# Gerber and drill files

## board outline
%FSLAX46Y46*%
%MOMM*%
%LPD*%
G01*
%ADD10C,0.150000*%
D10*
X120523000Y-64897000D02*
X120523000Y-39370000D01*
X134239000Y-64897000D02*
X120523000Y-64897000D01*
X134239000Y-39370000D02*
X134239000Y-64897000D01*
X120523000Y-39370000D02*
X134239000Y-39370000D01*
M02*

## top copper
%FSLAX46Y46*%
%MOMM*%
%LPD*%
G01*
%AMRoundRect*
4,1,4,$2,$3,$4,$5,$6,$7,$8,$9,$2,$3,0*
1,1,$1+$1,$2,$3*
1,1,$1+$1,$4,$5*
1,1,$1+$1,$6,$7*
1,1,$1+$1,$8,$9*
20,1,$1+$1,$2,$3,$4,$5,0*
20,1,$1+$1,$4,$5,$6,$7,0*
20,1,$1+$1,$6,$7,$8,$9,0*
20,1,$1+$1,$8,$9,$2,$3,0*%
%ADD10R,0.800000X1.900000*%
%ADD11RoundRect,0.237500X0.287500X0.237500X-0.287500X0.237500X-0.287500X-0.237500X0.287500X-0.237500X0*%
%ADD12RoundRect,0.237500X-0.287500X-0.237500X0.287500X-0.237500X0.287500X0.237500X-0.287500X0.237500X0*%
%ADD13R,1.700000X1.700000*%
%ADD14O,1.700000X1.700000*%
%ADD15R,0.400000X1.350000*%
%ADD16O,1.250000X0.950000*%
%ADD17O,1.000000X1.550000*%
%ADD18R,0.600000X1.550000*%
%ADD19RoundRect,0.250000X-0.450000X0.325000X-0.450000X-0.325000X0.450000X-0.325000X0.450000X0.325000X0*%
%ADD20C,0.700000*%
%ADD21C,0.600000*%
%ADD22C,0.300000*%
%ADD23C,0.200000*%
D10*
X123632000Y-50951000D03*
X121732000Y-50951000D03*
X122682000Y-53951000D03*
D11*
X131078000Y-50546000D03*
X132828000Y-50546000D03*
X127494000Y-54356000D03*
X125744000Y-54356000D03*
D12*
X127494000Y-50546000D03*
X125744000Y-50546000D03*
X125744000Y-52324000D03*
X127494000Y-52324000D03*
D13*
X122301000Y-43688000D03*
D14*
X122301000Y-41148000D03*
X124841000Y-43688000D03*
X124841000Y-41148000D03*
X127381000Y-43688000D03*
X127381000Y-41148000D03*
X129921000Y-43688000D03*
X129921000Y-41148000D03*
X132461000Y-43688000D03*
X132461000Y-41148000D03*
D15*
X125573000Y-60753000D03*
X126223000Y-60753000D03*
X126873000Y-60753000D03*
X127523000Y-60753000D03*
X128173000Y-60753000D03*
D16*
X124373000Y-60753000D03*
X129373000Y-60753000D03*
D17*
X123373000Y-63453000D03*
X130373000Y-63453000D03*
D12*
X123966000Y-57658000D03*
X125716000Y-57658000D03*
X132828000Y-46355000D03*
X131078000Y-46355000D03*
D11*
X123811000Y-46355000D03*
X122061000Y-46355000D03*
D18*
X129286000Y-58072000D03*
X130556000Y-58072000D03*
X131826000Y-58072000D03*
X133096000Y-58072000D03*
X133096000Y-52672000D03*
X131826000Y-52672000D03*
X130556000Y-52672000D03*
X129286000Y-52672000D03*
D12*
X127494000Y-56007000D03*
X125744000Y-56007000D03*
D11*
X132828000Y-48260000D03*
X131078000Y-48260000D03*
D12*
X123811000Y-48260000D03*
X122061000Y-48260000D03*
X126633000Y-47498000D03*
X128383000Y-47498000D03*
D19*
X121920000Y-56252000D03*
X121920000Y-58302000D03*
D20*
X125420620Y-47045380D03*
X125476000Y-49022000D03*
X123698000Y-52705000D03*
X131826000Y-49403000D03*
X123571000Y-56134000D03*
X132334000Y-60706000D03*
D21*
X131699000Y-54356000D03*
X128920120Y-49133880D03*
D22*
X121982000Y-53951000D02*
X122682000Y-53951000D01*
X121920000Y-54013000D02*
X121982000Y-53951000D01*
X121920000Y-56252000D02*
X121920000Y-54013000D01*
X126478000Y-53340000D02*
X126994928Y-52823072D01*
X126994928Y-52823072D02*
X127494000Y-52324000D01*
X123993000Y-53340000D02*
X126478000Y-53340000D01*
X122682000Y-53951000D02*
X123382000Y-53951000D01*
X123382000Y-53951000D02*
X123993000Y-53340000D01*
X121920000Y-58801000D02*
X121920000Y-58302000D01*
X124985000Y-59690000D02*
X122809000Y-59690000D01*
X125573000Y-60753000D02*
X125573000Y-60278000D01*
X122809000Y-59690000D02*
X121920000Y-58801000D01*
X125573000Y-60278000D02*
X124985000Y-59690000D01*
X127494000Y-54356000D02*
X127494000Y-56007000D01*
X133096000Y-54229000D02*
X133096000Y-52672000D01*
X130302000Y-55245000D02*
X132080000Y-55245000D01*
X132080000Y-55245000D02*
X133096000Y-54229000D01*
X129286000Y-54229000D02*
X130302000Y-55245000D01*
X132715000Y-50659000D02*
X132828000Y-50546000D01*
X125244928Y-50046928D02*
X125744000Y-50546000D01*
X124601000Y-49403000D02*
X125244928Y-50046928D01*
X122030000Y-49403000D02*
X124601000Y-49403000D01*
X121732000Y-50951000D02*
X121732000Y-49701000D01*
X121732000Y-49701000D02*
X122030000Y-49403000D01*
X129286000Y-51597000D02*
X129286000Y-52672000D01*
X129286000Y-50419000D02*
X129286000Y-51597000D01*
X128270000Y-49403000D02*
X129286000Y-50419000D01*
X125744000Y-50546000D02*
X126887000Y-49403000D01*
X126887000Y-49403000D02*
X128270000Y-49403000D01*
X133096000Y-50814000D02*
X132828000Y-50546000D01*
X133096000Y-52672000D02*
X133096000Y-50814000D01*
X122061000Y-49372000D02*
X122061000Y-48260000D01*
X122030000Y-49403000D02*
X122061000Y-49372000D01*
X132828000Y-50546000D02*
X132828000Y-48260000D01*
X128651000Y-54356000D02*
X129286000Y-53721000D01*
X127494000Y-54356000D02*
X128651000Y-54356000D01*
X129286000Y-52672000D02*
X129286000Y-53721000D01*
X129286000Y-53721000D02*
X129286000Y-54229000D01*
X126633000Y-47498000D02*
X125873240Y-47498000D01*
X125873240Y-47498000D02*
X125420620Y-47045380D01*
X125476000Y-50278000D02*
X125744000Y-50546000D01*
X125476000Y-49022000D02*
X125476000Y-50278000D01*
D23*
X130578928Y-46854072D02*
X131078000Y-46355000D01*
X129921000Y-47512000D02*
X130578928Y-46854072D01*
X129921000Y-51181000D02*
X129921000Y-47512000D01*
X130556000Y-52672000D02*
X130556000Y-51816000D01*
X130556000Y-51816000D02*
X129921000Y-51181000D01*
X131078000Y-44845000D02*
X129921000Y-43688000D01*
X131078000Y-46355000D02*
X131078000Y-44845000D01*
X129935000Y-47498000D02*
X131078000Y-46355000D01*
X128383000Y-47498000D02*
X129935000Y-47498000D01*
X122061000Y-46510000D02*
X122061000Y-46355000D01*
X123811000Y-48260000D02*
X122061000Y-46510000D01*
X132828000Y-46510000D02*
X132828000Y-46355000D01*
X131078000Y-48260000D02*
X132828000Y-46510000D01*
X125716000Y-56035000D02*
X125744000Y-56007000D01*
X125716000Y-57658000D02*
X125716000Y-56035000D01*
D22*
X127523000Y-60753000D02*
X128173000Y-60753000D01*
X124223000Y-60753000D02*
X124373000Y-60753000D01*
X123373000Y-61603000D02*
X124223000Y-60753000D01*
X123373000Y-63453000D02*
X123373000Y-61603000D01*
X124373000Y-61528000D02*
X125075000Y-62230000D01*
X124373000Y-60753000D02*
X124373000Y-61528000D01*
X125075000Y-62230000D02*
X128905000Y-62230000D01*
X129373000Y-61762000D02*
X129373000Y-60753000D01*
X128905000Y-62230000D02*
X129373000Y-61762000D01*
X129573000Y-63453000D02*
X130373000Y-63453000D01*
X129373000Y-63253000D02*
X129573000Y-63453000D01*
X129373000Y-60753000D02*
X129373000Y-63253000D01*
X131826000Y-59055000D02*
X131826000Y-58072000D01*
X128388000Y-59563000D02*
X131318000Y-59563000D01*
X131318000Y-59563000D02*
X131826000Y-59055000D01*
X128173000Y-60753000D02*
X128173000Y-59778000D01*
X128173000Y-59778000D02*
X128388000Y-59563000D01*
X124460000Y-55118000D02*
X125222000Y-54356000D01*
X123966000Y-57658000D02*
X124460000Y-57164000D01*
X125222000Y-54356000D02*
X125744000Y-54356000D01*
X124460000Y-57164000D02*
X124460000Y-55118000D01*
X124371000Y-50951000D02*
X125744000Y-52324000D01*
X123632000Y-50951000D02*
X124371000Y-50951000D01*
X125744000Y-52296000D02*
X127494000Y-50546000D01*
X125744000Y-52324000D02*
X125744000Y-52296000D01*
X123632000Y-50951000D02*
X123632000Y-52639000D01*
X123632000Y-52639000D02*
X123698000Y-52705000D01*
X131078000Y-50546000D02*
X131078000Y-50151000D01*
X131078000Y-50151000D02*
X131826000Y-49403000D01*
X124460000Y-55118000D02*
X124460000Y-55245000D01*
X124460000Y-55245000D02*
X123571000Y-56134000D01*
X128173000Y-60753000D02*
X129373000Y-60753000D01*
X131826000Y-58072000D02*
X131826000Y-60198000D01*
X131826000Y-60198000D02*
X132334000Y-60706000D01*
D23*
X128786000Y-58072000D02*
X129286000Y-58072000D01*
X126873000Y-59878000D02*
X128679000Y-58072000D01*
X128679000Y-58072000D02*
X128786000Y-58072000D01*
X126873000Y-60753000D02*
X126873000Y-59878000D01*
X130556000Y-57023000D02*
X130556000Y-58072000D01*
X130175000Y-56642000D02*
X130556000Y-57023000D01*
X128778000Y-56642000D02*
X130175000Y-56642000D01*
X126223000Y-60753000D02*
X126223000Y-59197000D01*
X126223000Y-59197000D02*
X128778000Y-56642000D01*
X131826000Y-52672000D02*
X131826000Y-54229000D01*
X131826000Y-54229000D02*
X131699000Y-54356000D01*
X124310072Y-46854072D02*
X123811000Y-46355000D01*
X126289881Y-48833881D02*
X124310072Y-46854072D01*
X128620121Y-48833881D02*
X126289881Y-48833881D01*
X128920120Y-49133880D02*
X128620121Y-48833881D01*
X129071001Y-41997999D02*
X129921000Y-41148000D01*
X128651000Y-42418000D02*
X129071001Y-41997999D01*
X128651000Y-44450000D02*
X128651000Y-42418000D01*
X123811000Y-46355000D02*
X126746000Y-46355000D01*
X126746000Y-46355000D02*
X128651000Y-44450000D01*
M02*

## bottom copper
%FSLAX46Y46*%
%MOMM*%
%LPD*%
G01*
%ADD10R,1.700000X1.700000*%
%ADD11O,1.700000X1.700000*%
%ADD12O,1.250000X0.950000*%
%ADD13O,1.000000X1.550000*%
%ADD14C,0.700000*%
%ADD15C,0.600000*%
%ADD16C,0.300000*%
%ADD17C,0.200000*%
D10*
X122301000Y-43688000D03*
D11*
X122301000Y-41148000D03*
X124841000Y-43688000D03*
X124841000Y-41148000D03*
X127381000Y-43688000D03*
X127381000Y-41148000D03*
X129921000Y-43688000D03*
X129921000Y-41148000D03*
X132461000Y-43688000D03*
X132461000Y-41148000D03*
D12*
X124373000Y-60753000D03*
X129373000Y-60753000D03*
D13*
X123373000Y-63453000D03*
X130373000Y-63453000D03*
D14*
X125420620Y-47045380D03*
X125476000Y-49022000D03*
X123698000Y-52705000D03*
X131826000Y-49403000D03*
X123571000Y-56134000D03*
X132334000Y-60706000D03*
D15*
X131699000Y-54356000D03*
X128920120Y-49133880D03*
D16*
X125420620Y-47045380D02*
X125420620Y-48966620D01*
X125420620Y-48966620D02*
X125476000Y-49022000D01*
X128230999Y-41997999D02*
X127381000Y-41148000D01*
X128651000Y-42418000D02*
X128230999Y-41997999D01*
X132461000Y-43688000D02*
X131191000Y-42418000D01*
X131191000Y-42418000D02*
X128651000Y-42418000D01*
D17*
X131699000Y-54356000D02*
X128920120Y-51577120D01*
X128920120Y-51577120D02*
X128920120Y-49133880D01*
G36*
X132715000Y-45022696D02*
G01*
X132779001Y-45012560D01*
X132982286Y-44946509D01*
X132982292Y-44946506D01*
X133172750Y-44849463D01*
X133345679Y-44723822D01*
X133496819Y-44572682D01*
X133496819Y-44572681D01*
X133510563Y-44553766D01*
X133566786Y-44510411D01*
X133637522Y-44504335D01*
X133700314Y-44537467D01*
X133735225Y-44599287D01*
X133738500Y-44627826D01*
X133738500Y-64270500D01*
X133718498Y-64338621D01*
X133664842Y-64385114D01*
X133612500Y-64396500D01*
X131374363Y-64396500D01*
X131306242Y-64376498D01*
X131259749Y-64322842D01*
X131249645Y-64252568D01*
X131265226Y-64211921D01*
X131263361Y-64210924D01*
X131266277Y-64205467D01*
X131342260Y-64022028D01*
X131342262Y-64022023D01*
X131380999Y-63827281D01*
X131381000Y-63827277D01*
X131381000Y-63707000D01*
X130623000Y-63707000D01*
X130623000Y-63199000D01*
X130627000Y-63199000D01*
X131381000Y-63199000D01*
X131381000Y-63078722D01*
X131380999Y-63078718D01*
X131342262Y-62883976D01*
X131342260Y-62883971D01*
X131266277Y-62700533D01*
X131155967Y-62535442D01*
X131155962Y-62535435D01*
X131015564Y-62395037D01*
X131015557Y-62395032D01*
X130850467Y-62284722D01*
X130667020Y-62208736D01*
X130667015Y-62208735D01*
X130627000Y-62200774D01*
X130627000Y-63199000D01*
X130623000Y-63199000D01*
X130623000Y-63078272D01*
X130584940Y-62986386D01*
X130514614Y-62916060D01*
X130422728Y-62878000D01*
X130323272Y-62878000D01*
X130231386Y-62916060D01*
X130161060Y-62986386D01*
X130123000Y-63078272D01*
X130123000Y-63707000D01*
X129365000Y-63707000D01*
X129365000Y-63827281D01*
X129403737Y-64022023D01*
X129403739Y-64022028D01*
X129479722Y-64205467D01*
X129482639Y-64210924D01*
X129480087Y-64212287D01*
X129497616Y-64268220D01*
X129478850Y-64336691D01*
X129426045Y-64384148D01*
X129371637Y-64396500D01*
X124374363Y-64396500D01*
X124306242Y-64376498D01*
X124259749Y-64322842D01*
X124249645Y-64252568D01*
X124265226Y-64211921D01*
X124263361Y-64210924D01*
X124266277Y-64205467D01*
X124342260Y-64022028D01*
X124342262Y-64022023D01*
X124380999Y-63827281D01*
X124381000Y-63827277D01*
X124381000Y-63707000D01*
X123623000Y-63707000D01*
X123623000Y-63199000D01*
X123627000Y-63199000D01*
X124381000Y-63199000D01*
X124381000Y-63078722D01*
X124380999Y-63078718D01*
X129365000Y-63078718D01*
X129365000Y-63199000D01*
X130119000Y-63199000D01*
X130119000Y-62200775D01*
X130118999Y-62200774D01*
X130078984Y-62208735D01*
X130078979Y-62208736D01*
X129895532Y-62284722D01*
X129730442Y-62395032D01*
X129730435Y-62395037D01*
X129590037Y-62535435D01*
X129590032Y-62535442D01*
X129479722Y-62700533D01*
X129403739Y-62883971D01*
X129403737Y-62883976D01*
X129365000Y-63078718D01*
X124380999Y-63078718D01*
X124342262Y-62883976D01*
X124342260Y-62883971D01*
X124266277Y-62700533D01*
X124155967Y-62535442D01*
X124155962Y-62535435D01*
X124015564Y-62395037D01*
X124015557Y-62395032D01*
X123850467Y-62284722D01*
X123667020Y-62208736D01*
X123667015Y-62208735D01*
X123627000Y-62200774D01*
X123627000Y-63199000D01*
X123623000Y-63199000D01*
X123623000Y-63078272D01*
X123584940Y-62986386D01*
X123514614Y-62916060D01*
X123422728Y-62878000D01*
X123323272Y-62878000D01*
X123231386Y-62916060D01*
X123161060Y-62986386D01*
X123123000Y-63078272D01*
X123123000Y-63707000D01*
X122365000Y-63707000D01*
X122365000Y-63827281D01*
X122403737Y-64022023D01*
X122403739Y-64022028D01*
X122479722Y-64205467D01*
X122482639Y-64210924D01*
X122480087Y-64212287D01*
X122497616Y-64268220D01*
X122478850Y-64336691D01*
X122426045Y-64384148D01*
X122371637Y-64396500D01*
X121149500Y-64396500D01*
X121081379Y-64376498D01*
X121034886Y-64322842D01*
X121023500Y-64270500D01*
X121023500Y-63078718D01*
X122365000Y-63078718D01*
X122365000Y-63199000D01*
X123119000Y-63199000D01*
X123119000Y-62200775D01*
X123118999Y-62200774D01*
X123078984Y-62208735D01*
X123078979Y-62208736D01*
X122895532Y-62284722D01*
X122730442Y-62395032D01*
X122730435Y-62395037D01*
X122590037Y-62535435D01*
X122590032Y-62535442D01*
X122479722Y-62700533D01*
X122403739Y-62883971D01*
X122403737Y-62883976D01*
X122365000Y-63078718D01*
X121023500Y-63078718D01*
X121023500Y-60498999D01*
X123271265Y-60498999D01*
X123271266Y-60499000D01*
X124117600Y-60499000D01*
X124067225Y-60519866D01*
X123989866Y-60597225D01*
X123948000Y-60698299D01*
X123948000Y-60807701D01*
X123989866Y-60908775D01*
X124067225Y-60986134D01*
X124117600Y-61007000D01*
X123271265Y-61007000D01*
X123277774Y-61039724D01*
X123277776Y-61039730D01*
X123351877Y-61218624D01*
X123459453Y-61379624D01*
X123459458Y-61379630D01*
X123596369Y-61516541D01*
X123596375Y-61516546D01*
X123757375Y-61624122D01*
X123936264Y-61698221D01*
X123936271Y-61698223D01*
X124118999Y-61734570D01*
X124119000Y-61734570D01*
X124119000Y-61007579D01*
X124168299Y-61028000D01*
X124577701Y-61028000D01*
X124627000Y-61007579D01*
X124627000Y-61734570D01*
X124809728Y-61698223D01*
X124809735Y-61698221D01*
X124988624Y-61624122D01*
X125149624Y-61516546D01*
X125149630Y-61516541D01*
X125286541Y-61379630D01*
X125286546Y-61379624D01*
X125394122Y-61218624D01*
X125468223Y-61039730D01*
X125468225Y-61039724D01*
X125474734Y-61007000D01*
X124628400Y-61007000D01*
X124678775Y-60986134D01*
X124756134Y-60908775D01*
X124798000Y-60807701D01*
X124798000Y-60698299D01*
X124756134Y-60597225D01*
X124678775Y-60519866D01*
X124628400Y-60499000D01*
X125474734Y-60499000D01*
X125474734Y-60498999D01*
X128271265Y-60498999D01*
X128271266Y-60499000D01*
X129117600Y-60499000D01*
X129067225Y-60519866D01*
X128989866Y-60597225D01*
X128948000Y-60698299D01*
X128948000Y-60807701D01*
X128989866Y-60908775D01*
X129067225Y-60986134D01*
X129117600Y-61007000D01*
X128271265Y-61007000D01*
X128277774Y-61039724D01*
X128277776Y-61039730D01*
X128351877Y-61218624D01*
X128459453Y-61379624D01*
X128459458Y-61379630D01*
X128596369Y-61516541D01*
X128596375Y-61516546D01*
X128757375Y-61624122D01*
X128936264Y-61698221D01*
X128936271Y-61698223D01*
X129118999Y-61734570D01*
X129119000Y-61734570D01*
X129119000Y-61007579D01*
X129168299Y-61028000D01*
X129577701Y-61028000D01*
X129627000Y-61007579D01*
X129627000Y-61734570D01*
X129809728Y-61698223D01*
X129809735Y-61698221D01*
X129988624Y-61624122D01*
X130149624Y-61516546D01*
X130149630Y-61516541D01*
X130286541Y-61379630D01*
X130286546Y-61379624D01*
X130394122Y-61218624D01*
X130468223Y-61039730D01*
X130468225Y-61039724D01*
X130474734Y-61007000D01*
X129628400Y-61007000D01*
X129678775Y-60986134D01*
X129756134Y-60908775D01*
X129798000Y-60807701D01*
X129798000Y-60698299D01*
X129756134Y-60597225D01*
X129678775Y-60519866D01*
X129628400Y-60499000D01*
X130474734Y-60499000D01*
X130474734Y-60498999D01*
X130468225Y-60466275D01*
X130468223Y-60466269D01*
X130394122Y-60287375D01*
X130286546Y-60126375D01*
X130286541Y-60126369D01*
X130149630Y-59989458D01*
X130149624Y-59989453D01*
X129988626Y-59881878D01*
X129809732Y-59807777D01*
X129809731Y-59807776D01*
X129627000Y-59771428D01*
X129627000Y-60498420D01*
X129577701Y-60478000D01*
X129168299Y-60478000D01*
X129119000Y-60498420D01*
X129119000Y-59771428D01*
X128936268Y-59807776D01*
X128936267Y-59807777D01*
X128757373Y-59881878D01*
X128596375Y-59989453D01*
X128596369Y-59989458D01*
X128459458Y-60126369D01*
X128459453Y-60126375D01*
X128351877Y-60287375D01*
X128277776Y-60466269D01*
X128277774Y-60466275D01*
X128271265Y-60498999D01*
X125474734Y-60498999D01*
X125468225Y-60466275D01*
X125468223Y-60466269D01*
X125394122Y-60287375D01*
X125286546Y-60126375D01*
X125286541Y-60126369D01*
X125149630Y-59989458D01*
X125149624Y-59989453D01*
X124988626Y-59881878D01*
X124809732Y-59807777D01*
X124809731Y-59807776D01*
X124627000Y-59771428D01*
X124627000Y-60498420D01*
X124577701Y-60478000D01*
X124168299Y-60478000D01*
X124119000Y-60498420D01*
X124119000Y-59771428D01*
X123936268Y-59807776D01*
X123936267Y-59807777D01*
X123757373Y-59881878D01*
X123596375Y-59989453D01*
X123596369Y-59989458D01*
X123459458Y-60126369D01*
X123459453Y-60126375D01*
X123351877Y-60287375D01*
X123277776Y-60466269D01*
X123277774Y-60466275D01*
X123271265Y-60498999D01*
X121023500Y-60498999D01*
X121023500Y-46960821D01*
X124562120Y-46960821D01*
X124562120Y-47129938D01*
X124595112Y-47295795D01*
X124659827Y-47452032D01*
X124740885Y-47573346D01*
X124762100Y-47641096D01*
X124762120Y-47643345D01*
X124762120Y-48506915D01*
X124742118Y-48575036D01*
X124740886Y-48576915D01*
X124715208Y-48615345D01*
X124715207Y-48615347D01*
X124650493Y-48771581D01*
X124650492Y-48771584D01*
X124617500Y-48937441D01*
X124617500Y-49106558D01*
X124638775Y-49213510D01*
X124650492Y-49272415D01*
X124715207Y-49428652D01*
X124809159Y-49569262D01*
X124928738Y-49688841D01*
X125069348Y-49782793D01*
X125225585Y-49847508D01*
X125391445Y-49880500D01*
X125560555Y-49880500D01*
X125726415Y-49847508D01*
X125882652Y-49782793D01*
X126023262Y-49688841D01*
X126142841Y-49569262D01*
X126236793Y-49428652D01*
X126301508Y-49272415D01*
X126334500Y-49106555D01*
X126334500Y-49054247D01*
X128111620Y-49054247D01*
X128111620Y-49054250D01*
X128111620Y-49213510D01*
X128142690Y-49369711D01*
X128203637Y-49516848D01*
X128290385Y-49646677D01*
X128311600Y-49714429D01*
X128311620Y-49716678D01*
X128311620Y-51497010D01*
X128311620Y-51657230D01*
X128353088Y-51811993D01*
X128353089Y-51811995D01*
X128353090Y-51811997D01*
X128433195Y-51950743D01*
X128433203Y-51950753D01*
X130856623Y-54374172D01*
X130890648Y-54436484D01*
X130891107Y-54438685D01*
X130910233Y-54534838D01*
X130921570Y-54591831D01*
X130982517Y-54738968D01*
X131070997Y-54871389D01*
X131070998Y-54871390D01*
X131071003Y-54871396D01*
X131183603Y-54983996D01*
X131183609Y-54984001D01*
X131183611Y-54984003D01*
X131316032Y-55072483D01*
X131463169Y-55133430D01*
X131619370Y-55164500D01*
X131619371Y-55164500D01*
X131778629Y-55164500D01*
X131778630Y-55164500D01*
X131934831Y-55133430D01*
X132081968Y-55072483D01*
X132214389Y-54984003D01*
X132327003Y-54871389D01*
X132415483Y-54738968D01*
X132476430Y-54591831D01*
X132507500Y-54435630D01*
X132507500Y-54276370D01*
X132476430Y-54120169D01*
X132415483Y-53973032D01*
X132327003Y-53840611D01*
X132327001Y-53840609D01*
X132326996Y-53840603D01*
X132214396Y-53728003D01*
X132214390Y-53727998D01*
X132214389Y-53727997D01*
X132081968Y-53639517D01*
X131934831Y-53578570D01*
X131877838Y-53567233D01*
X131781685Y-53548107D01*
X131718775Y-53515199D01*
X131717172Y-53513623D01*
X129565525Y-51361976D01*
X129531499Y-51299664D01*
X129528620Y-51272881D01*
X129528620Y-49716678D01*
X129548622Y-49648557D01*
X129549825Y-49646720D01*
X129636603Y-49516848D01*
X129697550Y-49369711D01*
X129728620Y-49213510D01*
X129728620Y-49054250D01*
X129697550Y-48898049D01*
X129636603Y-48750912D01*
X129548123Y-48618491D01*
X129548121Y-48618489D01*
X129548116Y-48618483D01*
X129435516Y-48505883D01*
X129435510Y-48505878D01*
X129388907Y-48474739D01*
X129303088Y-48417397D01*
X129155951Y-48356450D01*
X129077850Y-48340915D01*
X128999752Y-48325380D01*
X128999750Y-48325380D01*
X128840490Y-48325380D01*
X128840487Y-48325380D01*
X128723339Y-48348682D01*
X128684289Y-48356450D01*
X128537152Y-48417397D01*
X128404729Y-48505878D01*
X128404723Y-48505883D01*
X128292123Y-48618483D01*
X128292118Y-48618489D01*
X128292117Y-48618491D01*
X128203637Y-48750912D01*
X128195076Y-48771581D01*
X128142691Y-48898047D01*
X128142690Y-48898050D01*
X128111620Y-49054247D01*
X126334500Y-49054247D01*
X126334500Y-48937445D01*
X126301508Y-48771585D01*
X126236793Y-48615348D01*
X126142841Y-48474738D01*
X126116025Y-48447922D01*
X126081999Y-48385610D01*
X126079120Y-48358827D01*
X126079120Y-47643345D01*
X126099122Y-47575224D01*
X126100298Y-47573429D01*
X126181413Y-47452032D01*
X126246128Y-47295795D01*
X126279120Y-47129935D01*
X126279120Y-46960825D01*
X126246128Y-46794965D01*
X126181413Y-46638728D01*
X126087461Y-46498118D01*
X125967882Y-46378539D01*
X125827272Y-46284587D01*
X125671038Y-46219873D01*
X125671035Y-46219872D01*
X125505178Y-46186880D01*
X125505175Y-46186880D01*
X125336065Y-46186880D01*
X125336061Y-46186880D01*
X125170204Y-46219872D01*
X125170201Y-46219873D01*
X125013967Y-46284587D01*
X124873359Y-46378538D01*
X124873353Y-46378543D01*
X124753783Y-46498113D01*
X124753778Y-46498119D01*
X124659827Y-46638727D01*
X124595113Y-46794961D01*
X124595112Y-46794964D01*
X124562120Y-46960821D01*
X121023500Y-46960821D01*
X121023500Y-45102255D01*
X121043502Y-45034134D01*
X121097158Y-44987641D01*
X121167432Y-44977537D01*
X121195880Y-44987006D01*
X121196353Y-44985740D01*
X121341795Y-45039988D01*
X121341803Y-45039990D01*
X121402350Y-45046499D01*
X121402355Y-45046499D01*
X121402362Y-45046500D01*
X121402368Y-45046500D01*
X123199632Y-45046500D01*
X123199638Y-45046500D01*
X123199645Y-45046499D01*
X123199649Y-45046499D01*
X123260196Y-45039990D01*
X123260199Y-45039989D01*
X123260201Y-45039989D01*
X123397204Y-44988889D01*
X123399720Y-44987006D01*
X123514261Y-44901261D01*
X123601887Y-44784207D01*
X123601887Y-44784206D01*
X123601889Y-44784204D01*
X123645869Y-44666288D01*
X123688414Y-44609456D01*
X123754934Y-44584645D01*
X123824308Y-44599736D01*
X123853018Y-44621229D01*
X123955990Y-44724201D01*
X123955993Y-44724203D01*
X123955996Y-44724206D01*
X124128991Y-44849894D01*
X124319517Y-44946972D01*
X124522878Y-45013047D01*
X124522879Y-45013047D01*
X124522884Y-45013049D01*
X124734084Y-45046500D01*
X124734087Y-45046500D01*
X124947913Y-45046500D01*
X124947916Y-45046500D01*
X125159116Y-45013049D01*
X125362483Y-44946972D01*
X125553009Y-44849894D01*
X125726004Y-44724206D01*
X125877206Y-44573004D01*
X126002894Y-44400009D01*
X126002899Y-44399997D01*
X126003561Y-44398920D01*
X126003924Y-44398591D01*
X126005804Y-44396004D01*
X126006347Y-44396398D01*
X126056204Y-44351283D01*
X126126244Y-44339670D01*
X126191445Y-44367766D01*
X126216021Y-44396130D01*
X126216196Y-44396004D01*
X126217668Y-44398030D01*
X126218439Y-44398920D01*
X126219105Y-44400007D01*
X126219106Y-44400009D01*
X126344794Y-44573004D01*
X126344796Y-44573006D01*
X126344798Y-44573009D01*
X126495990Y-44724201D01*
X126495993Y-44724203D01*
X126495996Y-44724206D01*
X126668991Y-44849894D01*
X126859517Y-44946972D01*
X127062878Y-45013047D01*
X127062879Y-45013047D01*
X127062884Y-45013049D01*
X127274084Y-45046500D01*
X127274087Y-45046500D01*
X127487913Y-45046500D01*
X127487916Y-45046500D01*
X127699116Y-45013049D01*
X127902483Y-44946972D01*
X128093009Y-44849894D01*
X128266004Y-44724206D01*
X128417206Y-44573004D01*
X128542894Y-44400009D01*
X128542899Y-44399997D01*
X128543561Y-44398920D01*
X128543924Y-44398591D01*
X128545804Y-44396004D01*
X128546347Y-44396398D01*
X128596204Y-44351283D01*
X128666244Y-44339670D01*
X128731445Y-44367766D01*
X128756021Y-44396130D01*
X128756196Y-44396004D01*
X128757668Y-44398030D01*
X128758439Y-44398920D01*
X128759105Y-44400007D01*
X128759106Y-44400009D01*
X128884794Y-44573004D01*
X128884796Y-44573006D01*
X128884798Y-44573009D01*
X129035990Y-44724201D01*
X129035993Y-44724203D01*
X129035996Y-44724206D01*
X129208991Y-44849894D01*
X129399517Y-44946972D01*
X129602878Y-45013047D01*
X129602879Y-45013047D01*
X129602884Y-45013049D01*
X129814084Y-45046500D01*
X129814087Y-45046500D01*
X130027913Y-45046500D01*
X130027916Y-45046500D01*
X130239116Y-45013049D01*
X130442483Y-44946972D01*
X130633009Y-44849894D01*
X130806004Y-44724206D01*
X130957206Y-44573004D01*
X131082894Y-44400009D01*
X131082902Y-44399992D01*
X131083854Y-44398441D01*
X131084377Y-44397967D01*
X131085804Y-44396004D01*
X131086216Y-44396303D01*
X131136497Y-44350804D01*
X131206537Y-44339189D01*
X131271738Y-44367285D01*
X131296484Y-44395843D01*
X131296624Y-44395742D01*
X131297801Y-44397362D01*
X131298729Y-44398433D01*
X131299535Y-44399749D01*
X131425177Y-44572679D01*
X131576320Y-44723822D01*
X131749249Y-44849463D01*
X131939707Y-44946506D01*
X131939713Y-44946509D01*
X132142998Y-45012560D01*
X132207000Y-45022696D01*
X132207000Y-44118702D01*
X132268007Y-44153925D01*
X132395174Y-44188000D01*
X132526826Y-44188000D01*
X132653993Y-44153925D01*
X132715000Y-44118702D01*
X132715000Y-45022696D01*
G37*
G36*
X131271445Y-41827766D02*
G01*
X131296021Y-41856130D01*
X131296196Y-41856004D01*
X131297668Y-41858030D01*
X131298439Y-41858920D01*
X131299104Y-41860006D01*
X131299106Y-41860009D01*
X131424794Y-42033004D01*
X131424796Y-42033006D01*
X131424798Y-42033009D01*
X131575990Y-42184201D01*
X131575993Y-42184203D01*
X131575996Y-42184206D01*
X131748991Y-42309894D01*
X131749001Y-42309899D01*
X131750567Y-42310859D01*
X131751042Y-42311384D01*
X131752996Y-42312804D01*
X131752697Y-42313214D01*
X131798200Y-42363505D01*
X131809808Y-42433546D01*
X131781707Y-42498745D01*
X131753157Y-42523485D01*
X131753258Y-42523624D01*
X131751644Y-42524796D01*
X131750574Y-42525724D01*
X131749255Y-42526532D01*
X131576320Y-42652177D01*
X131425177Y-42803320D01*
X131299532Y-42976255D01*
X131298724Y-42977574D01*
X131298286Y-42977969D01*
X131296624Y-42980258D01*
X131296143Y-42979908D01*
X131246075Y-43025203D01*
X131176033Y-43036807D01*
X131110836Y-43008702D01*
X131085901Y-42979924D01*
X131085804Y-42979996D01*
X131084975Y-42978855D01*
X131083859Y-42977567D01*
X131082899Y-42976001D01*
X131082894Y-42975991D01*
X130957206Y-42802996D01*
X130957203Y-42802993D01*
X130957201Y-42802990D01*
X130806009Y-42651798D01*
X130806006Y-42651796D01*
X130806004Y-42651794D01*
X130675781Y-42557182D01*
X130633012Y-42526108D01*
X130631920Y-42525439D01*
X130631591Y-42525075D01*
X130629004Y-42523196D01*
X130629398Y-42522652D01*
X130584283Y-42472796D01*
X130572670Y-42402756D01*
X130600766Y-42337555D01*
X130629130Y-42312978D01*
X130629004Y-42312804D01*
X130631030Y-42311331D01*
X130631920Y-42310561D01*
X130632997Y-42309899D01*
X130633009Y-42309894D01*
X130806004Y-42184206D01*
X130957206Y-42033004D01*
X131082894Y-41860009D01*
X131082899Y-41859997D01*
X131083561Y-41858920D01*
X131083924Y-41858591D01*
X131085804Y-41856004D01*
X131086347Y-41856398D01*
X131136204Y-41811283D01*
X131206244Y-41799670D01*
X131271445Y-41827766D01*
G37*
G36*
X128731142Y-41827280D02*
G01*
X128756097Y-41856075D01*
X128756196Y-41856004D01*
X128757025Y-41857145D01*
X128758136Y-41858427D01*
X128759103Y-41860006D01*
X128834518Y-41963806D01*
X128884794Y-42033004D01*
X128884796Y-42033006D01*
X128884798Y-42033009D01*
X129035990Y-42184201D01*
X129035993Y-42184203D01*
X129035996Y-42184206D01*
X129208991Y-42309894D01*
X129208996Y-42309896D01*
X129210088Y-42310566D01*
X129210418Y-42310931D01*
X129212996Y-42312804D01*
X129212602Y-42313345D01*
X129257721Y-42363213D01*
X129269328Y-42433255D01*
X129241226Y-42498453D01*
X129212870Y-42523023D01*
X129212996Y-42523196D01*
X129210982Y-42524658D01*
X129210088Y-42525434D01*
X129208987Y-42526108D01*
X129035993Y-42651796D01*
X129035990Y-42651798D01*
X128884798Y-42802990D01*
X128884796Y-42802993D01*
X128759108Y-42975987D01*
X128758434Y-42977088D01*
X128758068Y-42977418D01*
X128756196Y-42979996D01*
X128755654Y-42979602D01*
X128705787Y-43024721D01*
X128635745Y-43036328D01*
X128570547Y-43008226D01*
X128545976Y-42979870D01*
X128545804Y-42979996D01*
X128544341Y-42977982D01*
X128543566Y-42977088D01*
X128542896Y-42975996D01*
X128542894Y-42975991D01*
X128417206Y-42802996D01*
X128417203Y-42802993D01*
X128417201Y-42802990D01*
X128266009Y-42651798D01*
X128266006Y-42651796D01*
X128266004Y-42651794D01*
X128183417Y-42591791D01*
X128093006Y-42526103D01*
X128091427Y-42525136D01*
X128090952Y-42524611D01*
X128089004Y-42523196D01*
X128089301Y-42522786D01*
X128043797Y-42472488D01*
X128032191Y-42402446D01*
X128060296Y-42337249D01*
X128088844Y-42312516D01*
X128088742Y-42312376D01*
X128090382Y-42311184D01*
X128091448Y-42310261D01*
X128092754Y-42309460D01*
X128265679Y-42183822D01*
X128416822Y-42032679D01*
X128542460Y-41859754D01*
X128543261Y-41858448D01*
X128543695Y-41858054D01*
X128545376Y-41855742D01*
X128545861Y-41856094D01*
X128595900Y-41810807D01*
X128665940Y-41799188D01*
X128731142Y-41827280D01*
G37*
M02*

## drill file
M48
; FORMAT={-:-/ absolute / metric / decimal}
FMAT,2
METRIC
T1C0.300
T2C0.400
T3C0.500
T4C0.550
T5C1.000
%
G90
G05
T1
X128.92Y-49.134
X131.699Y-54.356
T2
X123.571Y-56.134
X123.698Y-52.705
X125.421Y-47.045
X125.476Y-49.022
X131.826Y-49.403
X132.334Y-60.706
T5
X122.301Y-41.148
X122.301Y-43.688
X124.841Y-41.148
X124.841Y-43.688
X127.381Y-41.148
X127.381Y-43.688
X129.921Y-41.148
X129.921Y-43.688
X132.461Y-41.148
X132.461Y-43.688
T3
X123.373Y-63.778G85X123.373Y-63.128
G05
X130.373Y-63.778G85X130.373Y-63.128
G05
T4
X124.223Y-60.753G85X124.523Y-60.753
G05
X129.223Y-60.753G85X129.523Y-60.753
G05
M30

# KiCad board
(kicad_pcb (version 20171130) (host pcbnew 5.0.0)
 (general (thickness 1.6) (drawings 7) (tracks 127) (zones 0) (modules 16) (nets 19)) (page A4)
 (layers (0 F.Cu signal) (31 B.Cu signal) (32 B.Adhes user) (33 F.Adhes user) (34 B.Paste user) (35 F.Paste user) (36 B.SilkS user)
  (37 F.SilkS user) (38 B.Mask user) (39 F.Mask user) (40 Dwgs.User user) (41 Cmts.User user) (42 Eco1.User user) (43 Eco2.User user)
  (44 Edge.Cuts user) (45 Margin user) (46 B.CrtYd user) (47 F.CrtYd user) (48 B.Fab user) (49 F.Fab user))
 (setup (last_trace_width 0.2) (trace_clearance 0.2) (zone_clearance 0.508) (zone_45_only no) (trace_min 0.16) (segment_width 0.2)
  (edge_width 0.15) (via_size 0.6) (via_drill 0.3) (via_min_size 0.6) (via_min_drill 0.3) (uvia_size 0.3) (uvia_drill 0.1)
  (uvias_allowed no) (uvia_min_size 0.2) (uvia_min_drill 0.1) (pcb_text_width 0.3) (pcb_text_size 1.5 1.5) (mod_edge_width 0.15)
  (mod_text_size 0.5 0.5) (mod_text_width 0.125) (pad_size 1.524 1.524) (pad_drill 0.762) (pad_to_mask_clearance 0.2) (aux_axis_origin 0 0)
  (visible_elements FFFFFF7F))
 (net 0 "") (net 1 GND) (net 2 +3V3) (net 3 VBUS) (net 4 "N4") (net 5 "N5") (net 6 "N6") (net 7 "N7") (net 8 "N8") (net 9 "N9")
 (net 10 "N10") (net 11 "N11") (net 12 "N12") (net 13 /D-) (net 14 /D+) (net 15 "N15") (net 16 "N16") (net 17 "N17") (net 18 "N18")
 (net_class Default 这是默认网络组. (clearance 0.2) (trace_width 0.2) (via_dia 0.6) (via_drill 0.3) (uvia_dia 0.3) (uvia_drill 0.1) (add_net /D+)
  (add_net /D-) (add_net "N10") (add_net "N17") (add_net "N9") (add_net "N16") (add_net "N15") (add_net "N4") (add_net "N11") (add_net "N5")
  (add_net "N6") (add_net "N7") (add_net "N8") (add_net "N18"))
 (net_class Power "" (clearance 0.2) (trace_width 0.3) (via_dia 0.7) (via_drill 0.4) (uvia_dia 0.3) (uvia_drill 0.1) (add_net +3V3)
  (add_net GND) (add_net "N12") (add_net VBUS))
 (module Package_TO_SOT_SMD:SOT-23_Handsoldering (layer F.Cu) (at 122.682 52.451 270)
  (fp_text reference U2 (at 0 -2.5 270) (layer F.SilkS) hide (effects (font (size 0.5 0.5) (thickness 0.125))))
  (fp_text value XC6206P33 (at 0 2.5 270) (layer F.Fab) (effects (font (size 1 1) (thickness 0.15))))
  (pad 1 smd rect (at -1.5 -0.95 270) (size 1.9 0.8) (layers F.Cu F.Paste F.Mask) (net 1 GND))
  (pad 2 smd rect (at -1.5 0.95 270) (size 1.9 0.8) (layers F.Cu F.Paste F.Mask) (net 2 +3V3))
  (pad 3 smd rect (at 1.5 0 270) (size 1.9 0.8) (layers F.Cu F.Paste F.Mask) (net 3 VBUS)))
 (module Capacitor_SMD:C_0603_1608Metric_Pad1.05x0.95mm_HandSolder (layer F.Cu) (at 131.953 50.546 180)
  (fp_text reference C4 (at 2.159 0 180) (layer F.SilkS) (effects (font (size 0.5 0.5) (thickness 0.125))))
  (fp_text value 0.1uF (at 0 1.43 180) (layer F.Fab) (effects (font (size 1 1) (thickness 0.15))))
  (pad 2 smd roundrect (at 0.875 0 180) (size 1.05 0.95) (layers F.Cu F.Paste F.Mask) (roundrect_rratio 0.25) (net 1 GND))
  (pad 1 smd roundrect (at -0.875 0 180) (size 1.05 0.95) (layers F.Cu F.Paste F.Mask) (roundrect_rratio 0.25) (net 2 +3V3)))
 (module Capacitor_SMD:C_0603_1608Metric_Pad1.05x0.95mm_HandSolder (layer F.Cu) (at 126.619 54.356 180)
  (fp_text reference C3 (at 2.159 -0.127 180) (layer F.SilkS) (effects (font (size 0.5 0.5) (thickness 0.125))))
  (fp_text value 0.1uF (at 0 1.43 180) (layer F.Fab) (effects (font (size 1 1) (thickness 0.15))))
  (pad 1 smd roundrect (at -0.875 0 180) (size 1.05 0.95) (layers F.Cu F.Paste F.Mask) (roundrect_rratio 0.25) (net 2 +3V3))
  (pad 2 smd roundrect (at 0.875 0 180) (size 1.05 0.95) (layers F.Cu F.Paste F.Mask) (roundrect_rratio 0.25) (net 1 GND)))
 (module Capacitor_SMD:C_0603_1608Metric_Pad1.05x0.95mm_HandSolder (layer F.Cu) (at 126.619 50.546)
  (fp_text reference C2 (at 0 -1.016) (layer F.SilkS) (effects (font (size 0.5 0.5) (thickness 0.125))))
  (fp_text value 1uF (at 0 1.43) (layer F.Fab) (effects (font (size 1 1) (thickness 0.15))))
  (pad 2 smd roundrect (at 0.875 0) (size 1.05 0.95) (layers F.Cu F.Paste F.Mask) (roundrect_rratio 0.25) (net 1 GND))
  (pad 1 smd roundrect (at -0.875 0) (size 1.05 0.95) (layers F.Cu F.Paste F.Mask) (roundrect_rratio 0.25) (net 2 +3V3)))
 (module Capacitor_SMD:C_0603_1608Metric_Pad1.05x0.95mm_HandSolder (layer F.Cu) (at 126.619 52.324)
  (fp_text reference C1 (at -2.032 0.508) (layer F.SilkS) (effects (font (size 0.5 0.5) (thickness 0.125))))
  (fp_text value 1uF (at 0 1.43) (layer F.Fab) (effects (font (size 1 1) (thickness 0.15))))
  (pad 1 smd roundrect (at -0.875 0) (size 1.05 0.95) (layers F.Cu F.Paste F.Mask) (roundrect_rratio 0.25) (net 1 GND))
  (pad 2 smd roundrect (at 0.875 0) (size 1.05 0.95) (layers F.Cu F.Paste F.Mask) (roundrect_rratio 0.25) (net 3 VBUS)))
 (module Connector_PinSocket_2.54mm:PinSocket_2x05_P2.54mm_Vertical (layer B.Cu) (at 122.301 43.688 270)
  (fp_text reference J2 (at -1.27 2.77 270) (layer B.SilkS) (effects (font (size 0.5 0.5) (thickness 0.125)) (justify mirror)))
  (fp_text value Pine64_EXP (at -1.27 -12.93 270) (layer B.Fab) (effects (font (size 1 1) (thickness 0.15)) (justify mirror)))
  (pad 1 thru_hole rect (at 0 0 270) (size 1.7 1.7) (drill 1) (layers *.Cu *.Mask) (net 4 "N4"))
  (pad 2 thru_hole oval (at -2.54 0 270) (size 1.7 1.7) (drill 1) (layers *.Cu *.Mask) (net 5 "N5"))
  (pad 3 thru_hole oval (at 0 -2.54 270) (size 1.7 1.7) (drill 1) (layers *.Cu *.Mask) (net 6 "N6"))
  (pad 4 thru_hole oval (at -2.54 -2.54 270) (size 1.7 1.7) (drill 1) (layers *.Cu *.Mask) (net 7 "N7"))
  (pad 5 thru_hole oval (at 0 -5.08 270) (size 1.7 1.7) (drill 1) (layers *.Cu *.Mask) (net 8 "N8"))
  (pad 6 thru_hole oval (at -2.54 -5.08 270) (size 1.7 1.7) (drill 1) (layers *.Cu *.Mask) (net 1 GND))
  (pad 7 thru_hole oval (at 0 -7.62 270) (size 1.7 1.7) (drill 1) (layers *.Cu *.Mask) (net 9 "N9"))
  (pad 8 thru_hole oval (at -2.54 -7.62 270) (size 1.7 1.7) (drill 1) (layers *.Cu *.Mask) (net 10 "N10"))
  (pad 9 thru_hole oval (at 0 -10.16 270) (size 1.7 1.7) (drill 1) (layers *.Cu *.Mask) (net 1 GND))
  (pad 10 thru_hole oval (at -2.54 -10.16 270) (size 1.7 1.7) (drill 1) (layers *.Cu *.Mask) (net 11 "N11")))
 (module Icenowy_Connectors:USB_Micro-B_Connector (layer F.Cu) (at 126.873 62.103)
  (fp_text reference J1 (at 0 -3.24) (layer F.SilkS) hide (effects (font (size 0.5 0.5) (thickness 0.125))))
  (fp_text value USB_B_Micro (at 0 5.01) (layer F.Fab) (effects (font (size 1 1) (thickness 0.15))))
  (pad 1 smd rect (at -1.3 -1.35 90) (size 1.35 0.4) (layers F.Cu F.Paste F.Mask) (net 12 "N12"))
  (pad 2 smd rect (at -0.65 -1.35 90) (size 1.35 0.4) (layers F.Cu F.Paste F.Mask) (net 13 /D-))
  (pad 3 smd rect (at 0 -1.35 90) (size 1.35 0.4) (layers F.Cu F.Paste F.Mask) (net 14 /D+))
  (pad 4 smd rect (at 0.65 -1.35 90) (size 1.35 0.4) (layers F.Cu F.Paste F.Mask) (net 1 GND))
  (pad 5 smd rect (at 1.3 -1.35 90) (size 1.35 0.4) (layers F.Cu F.Paste F.Mask) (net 1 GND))
  (pad 6 thru_hole oval (at -2.5 -1.35 90) (size 0.95 1.25) (drill oval 0.55 0.85) (layers *.Cu *.Mask) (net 1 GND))
  (pad 6 thru_hole oval (at 2.5 -1.35 90) (size 0.95 1.25) (drill oval 0.55 0.85) (layers *.Cu *.Mask) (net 1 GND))
  (pad 6 thru_hole oval (at -3.5 1.35 90) (size 1.55 1) (drill oval 1.15 0.5) (layers *.Cu *.Mask) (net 1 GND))
  (pad 6 thru_hole oval (at 3.5 1.35 90) (size 1.55 1) (drill oval 1.15 0.5) (layers *.Cu *.Mask) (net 1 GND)))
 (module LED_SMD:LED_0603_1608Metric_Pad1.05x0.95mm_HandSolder (layer F.Cu) (at 124.841 57.658)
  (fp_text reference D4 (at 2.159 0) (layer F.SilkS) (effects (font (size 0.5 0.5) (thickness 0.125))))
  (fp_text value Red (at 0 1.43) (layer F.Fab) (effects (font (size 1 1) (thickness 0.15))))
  (pad 1 smd roundrect (at -0.875 0) (size 1.05 0.95) (layers F.Cu F.Paste F.Mask) (roundrect_rratio 0.25) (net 1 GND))
  (pad 2 smd roundrect (at 0.875 0) (size 1.05 0.95) (layers F.Cu F.Paste F.Mask) (roundrect_rratio 0.25) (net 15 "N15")))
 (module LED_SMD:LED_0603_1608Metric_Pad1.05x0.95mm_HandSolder (layer F.Cu) (at 131.953 46.355)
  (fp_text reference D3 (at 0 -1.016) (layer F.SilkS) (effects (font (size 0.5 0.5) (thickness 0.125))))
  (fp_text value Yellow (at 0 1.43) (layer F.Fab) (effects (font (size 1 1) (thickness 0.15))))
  (pad 2 smd roundrect (at 0.875 0) (size 1.05 0.95) (layers F.Cu F.Paste F.Mask) (roundrect_rratio 0.25) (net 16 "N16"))
  (pad 1 smd roundrect (at -0.875 0) (size 1.05 0.95) (layers F.Cu F.Paste F.Mask) (roundrect_rratio 0.25) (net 9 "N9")))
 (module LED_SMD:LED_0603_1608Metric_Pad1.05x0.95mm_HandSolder (layer F.Cu) (at 122.936 46.355 180)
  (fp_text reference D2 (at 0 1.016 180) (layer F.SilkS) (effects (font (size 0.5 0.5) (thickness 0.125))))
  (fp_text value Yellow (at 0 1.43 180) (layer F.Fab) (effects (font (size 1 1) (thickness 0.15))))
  (pad 1 smd roundrect (at -0.875 0 180) (size 1.05 0.95) (layers F.Cu F.Paste F.Mask) (roundrect_rratio 0.25) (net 10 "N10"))
  (pad 2 smd roundrect (at 0.875 0 180) (size 1.05 0.95) (layers F.Cu F.Paste F.Mask) (roundrect_rratio 0.25) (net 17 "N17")))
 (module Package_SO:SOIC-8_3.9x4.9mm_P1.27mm (layer F.Cu) (at 131.191 55.372 90)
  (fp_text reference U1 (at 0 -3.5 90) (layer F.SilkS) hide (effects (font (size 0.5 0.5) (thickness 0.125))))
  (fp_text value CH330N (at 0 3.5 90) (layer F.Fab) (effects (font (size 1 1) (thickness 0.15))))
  (pad 1 smd rect (at -2.7 -1.905 90) (size 1.55 0.6) (layers F.Cu F.Paste F.Mask) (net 14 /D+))
  (pad 2 smd rect (at -2.7 -0.635 90) (size 1.55 0.6) (layers F.Cu F.Paste F.Mask) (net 13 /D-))
  (pad 3 smd rect (at -2.7 0.635 90) (size 1.55 0.6) (layers F.Cu F.Paste F.Mask) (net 1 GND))
  (pad 4 smd rect (at -2.7 1.905 90) (size 1.55 0.6) (layers F.Cu F.Paste F.Mask) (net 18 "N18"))
  (pad 5 smd rect (at 2.7 1.905 90) (size 1.55 0.6) (layers F.Cu F.Paste F.Mask) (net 2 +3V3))
  (pad 6 smd rect (at 2.7 0.635 90) (size 1.55 0.6) (layers F.Cu F.Paste F.Mask) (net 10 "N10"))
  (pad 7 smd rect (at 2.7 -0.635 90) (size 1.55 0.6) (layers F.Cu F.Paste F.Mask) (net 9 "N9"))
  (pad 8 smd rect (at 2.7 -1.905 90) (size 1.55 0.6) (layers F.Cu F.Paste F.Mask) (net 2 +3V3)))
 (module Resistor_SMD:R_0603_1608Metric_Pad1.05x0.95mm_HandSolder (layer F.Cu) (at 126.619 56.007)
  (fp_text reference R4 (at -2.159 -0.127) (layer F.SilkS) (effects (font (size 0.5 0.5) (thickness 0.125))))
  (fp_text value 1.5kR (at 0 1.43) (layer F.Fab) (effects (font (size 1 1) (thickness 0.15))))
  (pad 2 smd roundrect (at 0.875 0) (size 1.05 0.95) (layers F.Cu F.Paste F.Mask) (roundrect_rratio 0.25) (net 2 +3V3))
  (pad 1 smd roundrect (at -0.875 0) (size 1.05 0.95) (layers F.Cu F.Paste F.Mask) (roundrect_rratio 0.25) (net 15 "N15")))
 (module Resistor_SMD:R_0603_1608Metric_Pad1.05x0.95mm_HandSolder (layer F.Cu) (at 131.953 48.26 180)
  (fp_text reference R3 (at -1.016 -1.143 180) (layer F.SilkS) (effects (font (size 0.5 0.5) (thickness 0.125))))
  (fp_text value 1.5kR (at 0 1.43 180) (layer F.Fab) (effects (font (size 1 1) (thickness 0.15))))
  (pad 1 smd roundrect (at -0.875 0 180) (size 1.05 0.95) (layers F.Cu F.Paste F.Mask) (roundrect_rratio 0.25) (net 2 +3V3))
  (pad 2 smd roundrect (at 0.875 0 180) (size 1.05 0.95) (layers F.Cu F.Paste F.Mask) (roundrect_rratio 0.25) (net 16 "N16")))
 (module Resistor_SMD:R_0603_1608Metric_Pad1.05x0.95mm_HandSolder (layer F.Cu) (at 122.936 48.26)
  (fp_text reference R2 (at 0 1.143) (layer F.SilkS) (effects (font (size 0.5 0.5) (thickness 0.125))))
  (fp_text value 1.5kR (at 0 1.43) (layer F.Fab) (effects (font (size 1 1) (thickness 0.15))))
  (pad 2 smd roundrect (at 0.875 0) (size 1.05 0.95) (layers F.Cu F.Paste F.Mask) (roundrect_rratio 0.25) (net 17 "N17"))
  (pad 1 smd roundrect (at -0.875 0) (size 1.05 0.95) (layers F.Cu F.Paste F.Mask) (roundrect_rratio 0.25) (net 2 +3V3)))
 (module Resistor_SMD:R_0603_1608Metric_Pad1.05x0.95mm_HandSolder (layer F.Cu) (at 127.508 47.498)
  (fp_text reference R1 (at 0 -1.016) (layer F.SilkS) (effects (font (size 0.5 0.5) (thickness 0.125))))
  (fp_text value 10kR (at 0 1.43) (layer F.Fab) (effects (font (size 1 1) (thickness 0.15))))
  (pad 1 smd roundrect (at -0.875 0) (size 1.05 0.95) (layers F.Cu F.Paste F.Mask) (roundrect_rratio 0.25) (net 2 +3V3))
  (pad 2 smd roundrect (at 0.875 0) (size 1.05 0.95) (layers F.Cu F.Paste F.Mask) (roundrect_rratio 0.25) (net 9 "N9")))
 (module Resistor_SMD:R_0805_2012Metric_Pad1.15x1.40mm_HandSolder (layer F.Cu) (at 121.92 57.277 270)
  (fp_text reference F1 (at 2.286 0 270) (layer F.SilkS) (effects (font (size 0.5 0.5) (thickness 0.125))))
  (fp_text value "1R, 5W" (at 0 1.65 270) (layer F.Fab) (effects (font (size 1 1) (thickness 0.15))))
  (pad 1 smd roundrect (at -1.025 0 270) (size 1.15 1.4) (layers F.Cu F.Paste F.Mask) (roundrect_rratio 0.217391) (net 3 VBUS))
  (pad 2 smd roundrect (at 1.025 0 270) (size 1.15 1.4) (layers F.Cu F.Paste F.Mask) (roundrect_rratio 0.217391) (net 12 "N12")))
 (gr_line (start 120.523 64.897) (end 120.523 39.37) (layer Edge.Cuts) (width 0.15))
 (gr_line (start 134.239 64.897) (end 120.523 64.897) (layer Edge.Cuts) (width 0.15))
 (gr_line (start 134.239 39.37) (end 134.239 64.897) (layer Edge.Cuts) (width 0.15))
 (gr_line (start 120.523 39.37) (end 134.239 39.37) (layer Edge.Cuts) (width 0.15))
 (segment (start 121.982 53.951) (end 122.682 53.951) (width 0.3) (layer F.Cu) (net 3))
 (segment (start 121.92 54.013) (end 121.982 53.951) (width 0.3) (layer F.Cu) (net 3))
 (segment (start 121.92 56.252) (end 121.92 54.013) (width 0.3) (layer F.Cu) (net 3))
 (segment (start 126.478 53.34) (end 126.994928 52.823072) (width 0.3) (layer F.Cu) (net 3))
 (segment (start 126.994928 52.823072) (end 127.494 52.324) (width 0.3) (layer F.Cu) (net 3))
 (segment (start 123.993 53.34) (end 126.478 53.34) (width 0.3) (layer F.Cu) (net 3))
 (segment (start 122.682 53.951) (end 123.382 53.951) (width 0.3) (layer F.Cu) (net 3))
 (segment (start 123.382 53.951) (end 123.993 53.34) (width 0.3) (layer F.Cu) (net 3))
 (segment (start 121.92 58.801) (end 121.92 58.302) (width 0.3) (layer F.Cu) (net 12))
 (segment (start 124.985 59.69) (end 122.809 59.69) (width 0.3) (layer F.Cu) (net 12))
 (segment (start 125.573 60.753) (end 125.573 60.278) (width 0.3) (layer F.Cu) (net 12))
 (segment (start 122.809 59.69) (end 121.92 58.801) (width 0.3) (layer F.Cu) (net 12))
 (segment (start 125.573 60.278) (end 124.985 59.69) (width 0.3) (layer F.Cu) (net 12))
 (segment (start 127.494 54.356) (end 127.494 56.007) (width 0.3) (layer F.Cu) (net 2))
 (segment (start 133.096 54.229) (end 133.096 52.672) (width 0.3) (layer F.Cu) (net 2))
 (segment (start 130.302 55.245) (end 132.08 55.245) (width 0.3) (layer F.Cu) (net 2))
 (segment (start 132.08 55.245) (end 133.096 54.229) (width 0.3) (layer F.Cu) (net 2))
 (segment (start 129.286 54.229) (end 130.302 55.245) (width 0.3) (layer F.Cu) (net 2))
 (segment (start 132.715 50.659) (end 132.828 50.546) (width 0.3) (layer F.Cu) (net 2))
 (segment (start 125.244928 50.046928) (end 125.744 50.546) (width 0.3) (layer F.Cu) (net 2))
 (segment (start 124.601 49.403) (end 125.244928 50.046928) (width 0.3) (layer F.Cu) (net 2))
 (segment (start 122.03 49.403) (end 124.601 49.403) (width 0.3) (layer F.Cu) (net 2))
 (segment (start 121.732 50.951) (end 121.732 49.701) (width 0.3) (layer F.Cu) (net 2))
 (segment (start 121.732 49.701) (end 122.03 49.403) (width 0.3) (layer F.Cu) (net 2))
 (segment (start 129.286 51.597) (end 129.286 52.672) (width 0.3) (layer F.Cu) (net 2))
 (segment (start 129.286 50.419) (end 129.286 51.597) (width 0.3) (layer F.Cu) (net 2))
 (segment (start 128.27 49.403) (end 129.286 50.419) (width 0.3) (layer F.Cu) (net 2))
 (segment (start 125.744 50.546) (end 126.887 49.403) (width 0.3) (layer F.Cu) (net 2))
 (segment (start 126.887 49.403) (end 128.27 49.403) (width 0.3) (layer F.Cu) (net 2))
 (segment (start 133.096 50.814) (end 132.828 50.546) (width 0.3) (layer F.Cu) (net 2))
 (segment (start 133.096 52.672) (end 133.096 50.814) (width 0.3) (layer F.Cu) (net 2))
 (segment (start 122.061 49.372) (end 122.061 48.26) (width 0.3) (layer F.Cu) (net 2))
 (segment (start 122.03 49.403) (end 122.061 49.372) (width 0.3) (layer F.Cu) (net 2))
 (segment (start 132.828 50.546) (end 132.828 48.26) (width 0.3) (layer F.Cu) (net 2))
 (segment (start 128.651 54.356) (end 129.286 53.721) (width 0.3) (layer F.Cu) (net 2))
 (segment (start 127.494 54.356) (end 128.651 54.356) (width 0.3) (layer F.Cu) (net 2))
 (segment (start 129.286 52.672) (end 129.286 53.721) (width 0.3) (layer F.Cu) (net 2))
 (segment (start 129.286 53.721) (end 129.286 54.229) (width 0.3) (layer F.Cu) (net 2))
 (via (at 125.42062 47.04538) (size 0.7) (drill 0.4) (layers F.Cu B.Cu) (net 2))
 (segment (start 126.633 47.498) (end 125.87324 47.498) (width 0.3) (layer F.Cu) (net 2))
 (segment (start 125.87324 47.498) (end 125.42062 47.04538) (width 0.3) (layer F.Cu) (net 2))
 (segment (start 125.42062 47.04538) (end 125.42062 48.96662) (width 0.3) (layer B.Cu) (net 2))
 (via (at 125.476 49.022) (size 0.7) (drill 0.4) (layers F.Cu B.Cu) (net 2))
 (segment (start 125.42062 48.96662) (end 125.476 49.022) (width 0.3) (layer B.Cu) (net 2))
 (segment (start 125.476 50.278) (end 125.744 50.546) (width 0.3) (layer F.Cu) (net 2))
 (segment (start 125.476 49.022) (end 125.476 50.278) (width 0.3) (layer F.Cu) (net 2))
 (segment (start 130.578928 46.854072) (end 131.078 46.355) (width 0.2) (layer F.Cu) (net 9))
 (segment (start 129.921 47.512) (end 130.578928 46.854072) (width 0.2) (layer F.Cu) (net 9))
 (segment (start 129.921 51.181) (end 129.921 47.512) (width 0.2) (layer F.Cu) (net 9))
 (segment (start 130.556 52.672) (end 130.556 51.816) (width 0.2) (layer F.Cu) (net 9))
 (segment (start 130.556 51.816) (end 129.921 51.181) (width 0.2) (layer F.Cu) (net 9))
 (segment (start 131.078 44.845) (end 129.921 43.688) (width 0.2) (layer F.Cu) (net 9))
 (segment (start 131.078 46.355) (end 131.078 44.845) (width 0.2) (layer F.Cu) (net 9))
 (segment (start 129.935 47.498) (end 131.078 46.355) (width 0.2) (layer F.Cu) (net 9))
 (segment (start 128.383 47.498) (end 129.935 47.498) (width 0.2) (layer F.Cu) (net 9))
 (segment (start 122.061 46.51) (end 122.061 46.355) (width 0.2) (layer F.Cu) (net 17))
 (segment (start 123.811 48.26) (end 122.061 46.51) (width 0.2) (layer F.Cu) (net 17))
 (segment (start 132.828 46.51) (end 132.828 46.355) (width 0.2) (layer F.Cu) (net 16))
 (segment (start 131.078 48.26) (end 132.828 46.51) (width 0.2) (layer F.Cu) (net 16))
 (segment (start 125.716 56.035) (end 125.744 56.007) (width 0.2) (layer F.Cu) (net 15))
 (segment (start 125.716 57.658) (end 125.716 56.035) (width 0.2) (layer F.Cu) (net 15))
 (segment (start 127.523 60.753) (end 128.173 60.753) (width 0.3) (layer F.Cu) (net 1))
 (segment (start 124.223 60.753) (end 124.373 60.753) (width 0.3) (layer F.Cu) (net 1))
 (segment (start 123.373 61.603) (end 124.223 60.753) (width 0.3) (layer F.Cu) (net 1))
 (segment (start 123.373 63.453) (end 123.373 61.603) (width 0.3) (layer F.Cu) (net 1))
 (segment (start 124.373 61.528) (end 125.075 62.23) (width 0.3) (layer F.Cu) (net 1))
 (segment (start 124.373 60.753) (end 124.373 61.528) (width 0.3) (layer F.Cu) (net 1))
 (segment (start 125.075 62.23) (end 128.905 62.23) (width 0.3) (layer F.Cu) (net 1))
 (segment (start 129.373 61.762) (end 129.373 60.753) (width 0.3) (layer F.Cu) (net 1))
 (segment (start 128.905 62.23) (end 129.373 61.762) (width 0.3) (layer F.Cu) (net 1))
 (segment (start 129.573 63.453) (end 130.373 63.453) (width 0.3) (layer F.Cu) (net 1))
 (segment (start 129.373 63.253) (end 129.573 63.453) (width 0.3) (layer F.Cu) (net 1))
 (segment (start 129.373 60.753) (end 129.373 63.253) (width 0.3) (layer F.Cu) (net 1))
 (segment (start 131.826 59.055) (end 131.826 58.072) (width 0.3) (layer F.Cu) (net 1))
 (segment (start 128.388 59.563) (end 131.318 59.563) (width 0.3) (layer F.Cu) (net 1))
 (segment (start 131.318 59.563) (end 131.826 59.055) (width 0.3) (layer F.Cu) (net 1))
 (segment (start 128.173 60.753) (end 128.173 59.778) (width 0.3) (layer F.Cu) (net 1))
 (segment (start 128.173 59.778) (end 128.388 59.563) (width 0.3) (layer F.Cu) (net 1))
 (segment (start 124.46 55.118) (end 125.222 54.356) (width 0.3) (layer F.Cu) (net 1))
 (segment (start 123.966 57.658) (end 124.46 57.164) (width 0.3) (layer F.Cu) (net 1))
 (segment (start 125.222 54.356) (end 125.744 54.356) (width 0.3) (layer F.Cu) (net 1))
 (segment (start 124.46 57.164) (end 124.46 55.118) (width 0.3) (layer F.Cu) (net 1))
 (segment (start 128.230999 41.997999) (end 127.381 41.148) (width 0.3) (layer B.Cu) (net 1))
 (segment (start 128.651 42.418) (end 128.230999 41.997999) (width 0.3) (layer B.Cu) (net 1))
 (segment (start 132.461 43.688) (end 131.191 42.418) (width 0.3) (layer B.Cu) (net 1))
 (segment (start 131.191 42.418) (end 128.651 42.418) (width 0.3) (layer B.Cu) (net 1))
 (segment (start 124.371 50.951) (end 125.744 52.324) (width 0.3) (layer F.Cu) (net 1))
 (segment (start 123.632 50.951) (end 124.371 50.951) (width 0.3) (layer F.Cu) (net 1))
 (segment (start 125.744 52.296) (end 127.494 50.546) (width 0.3) (layer F.Cu) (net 1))
 (segment (start 125.744 52.324) (end 125.744 52.296) (width 0.3) (layer F.Cu) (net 1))
 (via (at 123.698 52.705) (size 0.7) (drill 0.4) (layers F.Cu B.Cu) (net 1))
 (segment (start 123.632 50.951) (end 123.632 52.639) (width 0.3) (layer F.Cu) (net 1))
 (segment (start 123.632 52.639) (end 123.698 52.705) (width 0.3) (layer F.Cu) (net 1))
 (via (at 131.826 49.403) (size 0.7) (drill 0.4) (layers F.Cu B.Cu) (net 1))
 (segment (start 131.078 50.546) (end 131.078 50.151) (width 0.3) (layer F.Cu) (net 1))
 (segment (start 131.078 50.151) (end 131.826 49.403) (width 0.3) (layer F.Cu) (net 1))
 (via (at 123.571 56.134) (size 0.7) (drill 0.4) (layers F.Cu B.Cu) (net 1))
 (segment (start 124.46 55.118) (end 124.46 55.245) (width 0.3) (layer F.Cu) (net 1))
 (segment (start 124.46 55.245) (end 123.571 56.134) (width 0.3) (layer F.Cu) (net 1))
 (segment (start 128.173 60.753) (end 129.373 60.753) (width 0.3) (layer F.Cu) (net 1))
 (via (at 132.334 60.706) (size 0.7) (drill 0.4) (layers F.Cu B.Cu) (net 1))
 (segment (start 131.826 58.072) (end 131.826 60.198) (width 0.3) (layer F.Cu) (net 1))
 (segment (start 131.826 60.198) (end 132.334 60.706) (width 0.3) (layer F.Cu) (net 1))
 (segment (start 128.786 58.072) (end 129.286 58.072) (width 0.2) (layer F.Cu) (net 14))
 (segment (start 126.873 59.878) (end 128.679 58.072) (width 0.2) (layer F.Cu) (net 14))
 (segment (start 128.679 58.072) (end 128.786 58.072) (width 0.2) (layer F.Cu) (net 14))
 (segment (start 126.873 60.753) (end 126.873 59.878) (width 0.2) (layer F.Cu) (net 14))
 (segment (start 130.556 57.023) (end 130.556 58.072) (width 0.2) (layer F.Cu) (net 13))
 (segment (start 130.175 56.642) (end 130.556 57.023) (width 0.2) (layer F.Cu) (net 13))
 (segment (start 128.778 56.642) (end 130.175 56.642) (width 0.2) (layer F.Cu) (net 13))
 (segment (start 126.223 60.753) (end 126.223 59.197) (width 0.2) (layer F.Cu) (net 13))
 (segment (start 126.223 59.197) (end 128.778 56.642) (width 0.2) (layer F.Cu) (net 13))
 (via (at 131.699 54.356) (size 0.6) (drill 0.3) (layers F.Cu B.Cu) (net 10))
 (segment (start 131.826 52.672) (end 131.826 54.229) (width 0.2) (layer F.Cu) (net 10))
 (segment (start 131.826 54.229) (end 131.699 54.356) (width 0.2) (layer F.Cu) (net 10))
 (via (at 128.92012 49.13388) (size 0.6) (drill 0.3) (layers F.Cu B.Cu) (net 10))
 (segment (start 131.699 54.356) (end 128.92012 51.57712) (width 0.2) (layer B.Cu) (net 10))
 (segment (start 128.92012 51.57712) (end 128.92012 49.13388) (width 0.2) (layer B.Cu) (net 10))
 (segment (start 124.310072 46.854072) (end 123.811 46.355) (width 0.2) (layer F.Cu) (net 10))
 (segment (start 126.289881 48.833881) (end 124.310072 46.854072) (width 0.2) (layer F.Cu) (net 10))
 (segment (start 128.620121 48.833881) (end 126.289881 48.833881) (width 0.2) (layer F.Cu) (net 10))
 (segment (start 128.92012 49.13388) (end 128.620121 48.833881) (width 0.2) (layer F.Cu) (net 10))
 (segment (start 129.071001 41.997999) (end 129.921 41.148) (width 0.2) (layer F.Cu) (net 10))
 (segment (start 128.651 42.418) (end 129.071001 41.997999) (width 0.2) (layer F.Cu) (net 10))
 (segment (start 128.651 44.45) (end 128.651 42.418) (width 0.2) (layer F.Cu) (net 10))
 (segment (start 123.811 46.355) (end 126.746 46.355) (width 0.2) (layer F.Cu) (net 10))
 (segment (start 126.746 46.355) (end 128.651 44.45) (width 0.2) (layer F.Cu) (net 10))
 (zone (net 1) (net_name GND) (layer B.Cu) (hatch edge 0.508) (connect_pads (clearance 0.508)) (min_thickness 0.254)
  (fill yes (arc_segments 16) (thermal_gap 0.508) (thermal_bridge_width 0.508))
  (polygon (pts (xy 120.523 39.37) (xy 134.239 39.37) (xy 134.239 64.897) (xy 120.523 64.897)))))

